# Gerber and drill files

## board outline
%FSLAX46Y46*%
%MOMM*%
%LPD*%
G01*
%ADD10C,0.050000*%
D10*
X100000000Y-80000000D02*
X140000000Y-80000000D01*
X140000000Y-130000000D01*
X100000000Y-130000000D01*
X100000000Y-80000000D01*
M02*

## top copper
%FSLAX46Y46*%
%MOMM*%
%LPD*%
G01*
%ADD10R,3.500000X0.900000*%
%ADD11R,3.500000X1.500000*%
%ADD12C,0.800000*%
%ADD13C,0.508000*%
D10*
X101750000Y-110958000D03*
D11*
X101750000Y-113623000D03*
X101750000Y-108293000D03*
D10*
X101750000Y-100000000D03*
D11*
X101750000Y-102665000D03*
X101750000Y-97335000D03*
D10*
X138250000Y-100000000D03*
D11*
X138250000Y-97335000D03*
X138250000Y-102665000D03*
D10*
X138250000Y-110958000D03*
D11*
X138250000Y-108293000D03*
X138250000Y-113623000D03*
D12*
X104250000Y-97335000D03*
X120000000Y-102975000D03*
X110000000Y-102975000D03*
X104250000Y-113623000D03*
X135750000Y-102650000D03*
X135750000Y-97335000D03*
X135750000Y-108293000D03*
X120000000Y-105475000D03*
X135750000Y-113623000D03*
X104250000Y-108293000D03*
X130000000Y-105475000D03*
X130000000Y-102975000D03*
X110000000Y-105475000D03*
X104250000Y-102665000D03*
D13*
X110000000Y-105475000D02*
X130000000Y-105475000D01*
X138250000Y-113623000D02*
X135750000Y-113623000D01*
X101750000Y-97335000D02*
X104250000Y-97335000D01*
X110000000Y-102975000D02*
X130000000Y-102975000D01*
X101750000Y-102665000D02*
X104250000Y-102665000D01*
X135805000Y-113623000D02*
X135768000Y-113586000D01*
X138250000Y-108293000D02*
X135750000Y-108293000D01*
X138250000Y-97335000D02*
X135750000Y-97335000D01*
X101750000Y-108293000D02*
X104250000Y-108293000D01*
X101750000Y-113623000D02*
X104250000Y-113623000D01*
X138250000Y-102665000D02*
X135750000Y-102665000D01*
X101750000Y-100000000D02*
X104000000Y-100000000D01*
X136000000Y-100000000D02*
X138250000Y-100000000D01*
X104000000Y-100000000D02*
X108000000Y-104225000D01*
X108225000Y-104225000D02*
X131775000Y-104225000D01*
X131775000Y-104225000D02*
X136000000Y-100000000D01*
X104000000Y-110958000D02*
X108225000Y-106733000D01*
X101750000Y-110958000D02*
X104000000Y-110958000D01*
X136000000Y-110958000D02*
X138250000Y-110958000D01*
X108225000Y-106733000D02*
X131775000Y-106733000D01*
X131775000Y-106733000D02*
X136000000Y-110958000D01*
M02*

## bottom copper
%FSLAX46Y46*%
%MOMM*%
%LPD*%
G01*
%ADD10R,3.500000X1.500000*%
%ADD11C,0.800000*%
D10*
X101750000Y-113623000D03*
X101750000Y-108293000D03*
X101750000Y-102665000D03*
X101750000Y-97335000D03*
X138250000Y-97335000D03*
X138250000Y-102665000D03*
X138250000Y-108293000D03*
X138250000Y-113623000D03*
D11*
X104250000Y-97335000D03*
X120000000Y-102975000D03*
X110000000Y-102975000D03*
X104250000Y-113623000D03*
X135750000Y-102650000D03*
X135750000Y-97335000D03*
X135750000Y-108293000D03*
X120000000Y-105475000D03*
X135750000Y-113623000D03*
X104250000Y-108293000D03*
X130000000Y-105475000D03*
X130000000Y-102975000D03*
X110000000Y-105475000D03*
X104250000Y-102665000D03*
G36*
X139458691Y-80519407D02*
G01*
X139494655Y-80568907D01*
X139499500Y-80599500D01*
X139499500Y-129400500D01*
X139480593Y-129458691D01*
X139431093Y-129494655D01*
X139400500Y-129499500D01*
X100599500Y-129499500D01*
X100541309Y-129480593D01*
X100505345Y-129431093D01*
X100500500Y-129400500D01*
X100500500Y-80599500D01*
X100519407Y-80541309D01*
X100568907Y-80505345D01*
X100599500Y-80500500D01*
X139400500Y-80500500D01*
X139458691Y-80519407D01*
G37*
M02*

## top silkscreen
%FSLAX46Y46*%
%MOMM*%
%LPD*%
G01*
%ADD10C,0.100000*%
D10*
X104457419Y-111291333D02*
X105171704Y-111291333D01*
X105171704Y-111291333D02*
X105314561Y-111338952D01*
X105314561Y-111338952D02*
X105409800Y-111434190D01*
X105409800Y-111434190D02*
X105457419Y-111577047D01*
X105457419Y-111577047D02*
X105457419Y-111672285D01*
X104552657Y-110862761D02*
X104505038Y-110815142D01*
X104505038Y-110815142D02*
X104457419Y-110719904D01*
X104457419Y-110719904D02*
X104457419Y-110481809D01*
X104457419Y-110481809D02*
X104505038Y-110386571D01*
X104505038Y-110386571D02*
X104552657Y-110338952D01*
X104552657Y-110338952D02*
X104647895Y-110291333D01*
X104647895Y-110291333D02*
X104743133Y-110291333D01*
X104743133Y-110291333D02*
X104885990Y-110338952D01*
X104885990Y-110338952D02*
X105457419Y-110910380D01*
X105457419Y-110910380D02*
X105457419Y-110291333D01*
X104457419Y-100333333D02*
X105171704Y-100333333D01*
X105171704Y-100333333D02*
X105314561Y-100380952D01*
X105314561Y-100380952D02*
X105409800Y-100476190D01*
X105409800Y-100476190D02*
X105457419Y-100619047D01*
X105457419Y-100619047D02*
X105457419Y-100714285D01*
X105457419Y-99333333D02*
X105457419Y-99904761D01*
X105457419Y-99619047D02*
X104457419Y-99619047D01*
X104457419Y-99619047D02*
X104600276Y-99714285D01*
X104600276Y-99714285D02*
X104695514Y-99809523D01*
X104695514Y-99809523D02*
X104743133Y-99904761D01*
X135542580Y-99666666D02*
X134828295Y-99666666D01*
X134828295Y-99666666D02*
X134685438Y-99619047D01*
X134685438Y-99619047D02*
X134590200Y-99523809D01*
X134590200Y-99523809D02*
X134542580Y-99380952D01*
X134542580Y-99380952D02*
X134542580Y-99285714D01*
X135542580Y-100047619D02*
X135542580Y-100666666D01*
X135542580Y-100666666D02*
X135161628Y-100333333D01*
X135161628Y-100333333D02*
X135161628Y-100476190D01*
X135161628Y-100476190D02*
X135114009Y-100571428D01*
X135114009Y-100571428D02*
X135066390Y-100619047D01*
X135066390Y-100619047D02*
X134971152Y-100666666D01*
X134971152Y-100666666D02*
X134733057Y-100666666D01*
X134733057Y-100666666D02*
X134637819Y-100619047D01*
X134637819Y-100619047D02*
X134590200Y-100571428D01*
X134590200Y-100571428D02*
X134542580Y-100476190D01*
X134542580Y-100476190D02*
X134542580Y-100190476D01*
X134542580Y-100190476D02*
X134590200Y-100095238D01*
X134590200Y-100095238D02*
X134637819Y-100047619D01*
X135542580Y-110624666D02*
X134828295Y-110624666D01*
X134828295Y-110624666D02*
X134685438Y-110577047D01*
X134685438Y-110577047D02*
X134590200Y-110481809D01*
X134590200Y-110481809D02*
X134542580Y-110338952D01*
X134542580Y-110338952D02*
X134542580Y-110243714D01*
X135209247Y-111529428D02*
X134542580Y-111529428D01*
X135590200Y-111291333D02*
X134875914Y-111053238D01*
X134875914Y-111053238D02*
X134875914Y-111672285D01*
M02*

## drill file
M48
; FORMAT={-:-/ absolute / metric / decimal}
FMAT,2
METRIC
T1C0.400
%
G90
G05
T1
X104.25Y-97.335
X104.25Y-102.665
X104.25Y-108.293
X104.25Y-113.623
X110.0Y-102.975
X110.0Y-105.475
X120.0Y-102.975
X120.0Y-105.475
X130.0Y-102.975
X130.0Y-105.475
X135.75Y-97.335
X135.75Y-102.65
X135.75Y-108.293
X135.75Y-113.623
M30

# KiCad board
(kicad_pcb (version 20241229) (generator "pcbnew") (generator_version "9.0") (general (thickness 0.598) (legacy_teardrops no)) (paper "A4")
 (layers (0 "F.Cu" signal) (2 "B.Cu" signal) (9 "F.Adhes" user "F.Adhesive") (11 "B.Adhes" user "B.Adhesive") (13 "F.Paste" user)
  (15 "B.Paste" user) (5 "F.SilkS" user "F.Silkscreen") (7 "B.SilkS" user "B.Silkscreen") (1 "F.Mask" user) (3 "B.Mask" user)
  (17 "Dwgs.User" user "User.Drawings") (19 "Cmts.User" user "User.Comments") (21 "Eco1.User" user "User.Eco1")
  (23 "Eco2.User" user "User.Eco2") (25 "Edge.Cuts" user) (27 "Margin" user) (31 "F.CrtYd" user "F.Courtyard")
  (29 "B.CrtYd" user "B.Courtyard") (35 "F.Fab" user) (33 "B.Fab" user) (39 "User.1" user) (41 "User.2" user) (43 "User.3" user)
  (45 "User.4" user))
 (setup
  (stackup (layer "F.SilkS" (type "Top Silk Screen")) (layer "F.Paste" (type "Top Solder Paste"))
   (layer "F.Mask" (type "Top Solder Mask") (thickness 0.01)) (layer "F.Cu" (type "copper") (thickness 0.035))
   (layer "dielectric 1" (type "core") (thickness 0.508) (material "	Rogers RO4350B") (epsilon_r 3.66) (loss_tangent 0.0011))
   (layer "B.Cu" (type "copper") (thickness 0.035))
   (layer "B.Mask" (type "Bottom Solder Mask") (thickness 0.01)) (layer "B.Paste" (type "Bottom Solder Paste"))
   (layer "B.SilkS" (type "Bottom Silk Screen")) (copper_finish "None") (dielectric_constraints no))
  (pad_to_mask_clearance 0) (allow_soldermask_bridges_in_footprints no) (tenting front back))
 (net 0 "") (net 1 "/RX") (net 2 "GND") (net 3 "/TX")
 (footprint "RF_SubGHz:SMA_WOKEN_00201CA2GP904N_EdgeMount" (layer "F.Cu") (at 100 110.958 90)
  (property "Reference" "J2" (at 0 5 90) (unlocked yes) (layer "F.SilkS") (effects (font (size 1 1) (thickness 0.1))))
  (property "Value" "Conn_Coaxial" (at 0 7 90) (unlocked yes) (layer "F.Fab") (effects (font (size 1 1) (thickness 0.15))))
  (pad "1" smd rect (at 0 1.75 90) (size 0.9 3.5) (layers "F.Cu" "F.Mask") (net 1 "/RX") (thermal_bridge_angle 45))
  (pad "2" smd rect (at -2.665 1.75 90) (size 1.5 3.5) (layers "F.Cu" "F.Mask") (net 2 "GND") (thermal_bridge_angle 45))
  (pad "2" smd rect (at -2.665 1.75 90) (size 1.5 3.5) (layers "B.Cu" "B.Mask") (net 2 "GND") (thermal_bridge_angle 45))
  (pad "2" smd rect (at 2.665 1.75 90) (size 1.5 3.5) (layers "F.Cu" "F.Mask") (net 2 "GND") (thermal_bridge_angle 45))
  (pad "2" smd rect (at 2.665 1.75 90) (size 1.5 3.5) (layers "B.Cu" "B.Mask") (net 2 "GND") (thermal_bridge_angle 45)))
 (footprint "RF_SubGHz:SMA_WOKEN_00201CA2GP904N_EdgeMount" (layer "F.Cu") (at 100 100 90)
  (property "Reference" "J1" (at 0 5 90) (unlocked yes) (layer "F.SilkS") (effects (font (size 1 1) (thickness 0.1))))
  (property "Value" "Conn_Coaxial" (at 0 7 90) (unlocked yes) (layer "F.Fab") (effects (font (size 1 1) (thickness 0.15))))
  (pad "1" smd rect (at 0 1.75 90) (size 0.9 3.5) (layers "F.Cu" "F.Mask") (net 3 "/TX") (thermal_bridge_angle 45))
  (pad "2" smd rect (at -2.665 1.75 90) (size 1.5 3.5) (layers "F.Cu" "F.Mask") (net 2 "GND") (thermal_bridge_angle 45))
  (pad "2" smd rect (at -2.665 1.75 90) (size 1.5 3.5) (layers "B.Cu" "B.Mask") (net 2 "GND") (thermal_bridge_angle 45))
  (pad "2" smd rect (at 2.665 1.75 90) (size 1.5 3.5) (layers "F.Cu" "F.Mask") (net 2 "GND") (thermal_bridge_angle 45))
  (pad "2" smd rect (at 2.665 1.75 90) (size 1.5 3.5) (layers "B.Cu" "B.Mask") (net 2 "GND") (thermal_bridge_angle 45)))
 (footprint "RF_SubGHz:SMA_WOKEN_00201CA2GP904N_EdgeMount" (layer "F.Cu") (at 140 100 -90)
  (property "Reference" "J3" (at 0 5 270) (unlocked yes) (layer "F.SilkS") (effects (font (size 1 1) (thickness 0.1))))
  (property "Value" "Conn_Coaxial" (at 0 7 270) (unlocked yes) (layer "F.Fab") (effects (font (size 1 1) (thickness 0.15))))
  (pad "1" smd rect (at 0 1.75 270) (size 0.9 3.5) (layers "F.Cu" "F.Mask") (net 3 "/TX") (thermal_bridge_angle 45))
  (pad "2" smd rect (at -2.665 1.75 270) (size 1.5 3.5) (layers "F.Cu" "F.Mask") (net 2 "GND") (thermal_bridge_angle 45))
  (pad "2" smd rect (at -2.665 1.75 270) (size 1.5 3.5) (layers "B.Cu" "B.Mask") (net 2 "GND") (thermal_bridge_angle 45))
  (pad "2" smd rect (at 2.665 1.75 270) (size 1.5 3.5) (layers "F.Cu" "F.Mask") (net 2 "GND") (thermal_bridge_angle 45))
  (pad "2" smd rect (at 2.665 1.75 270) (size 1.5 3.5) (layers "B.Cu" "B.Mask") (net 2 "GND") (thermal_bridge_angle 45)))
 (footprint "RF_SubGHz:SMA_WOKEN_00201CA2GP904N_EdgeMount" (layer "F.Cu") (at 140 110.958 -90)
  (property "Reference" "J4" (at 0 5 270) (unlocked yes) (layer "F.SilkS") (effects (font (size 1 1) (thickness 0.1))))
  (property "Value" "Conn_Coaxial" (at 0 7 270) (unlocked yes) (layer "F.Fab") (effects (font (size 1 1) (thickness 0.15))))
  (pad "1" smd rect (at 0 1.75 270) (size 0.9 3.5) (layers "F.Cu" "F.Mask") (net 1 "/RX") (thermal_bridge_angle 45))
  (pad "2" smd rect (at -2.665 1.75 270) (size 1.5 3.5) (layers "F.Cu" "F.Mask") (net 2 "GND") (thermal_bridge_angle 45))
  (pad "2" smd rect (at -2.665 1.75 270) (size 1.5 3.5) (layers "B.Cu" "B.Mask") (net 2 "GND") (thermal_bridge_angle 45))
  (pad "2" smd rect (at 2.665 1.75 270) (size 1.5 3.5) (layers "F.Cu" "F.Mask") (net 2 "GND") (thermal_bridge_angle 45))
  (pad "2" smd rect (at 2.665 1.75 270) (size 1.5 3.5) (layers "B.Cu" "B.Mask") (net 2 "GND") (thermal_bridge_angle 45)))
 (gr_rect (start 100 80) (end 140 130) (stroke (width 0.05) (type solid)) (fill no) (layer "Edge.Cuts"))
 (segment (start 110 105.475) (end 130 105.475) (width 0.508) (layer "F.Cu") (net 2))
 (segment (start 138.25 113.623) (end 135.75 113.623) (width 0.508) (layer "F.Cu") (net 2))
 (segment (start 101.75 97.335) (end 104.25 97.335) (width 0.508) (layer "F.Cu") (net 2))
 (segment (start 110 102.975) (end 130 102.975) (width 0.508) (layer "F.Cu") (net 2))
 (segment (start 101.75 102.665) (end 104.25 102.665) (width 0.508) (layer "F.Cu") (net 2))
 (segment (start 135.805 113.623) (end 135.768 113.586) (width 0.508) (layer "F.Cu") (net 2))
 (segment (start 138.25 108.293) (end 135.75 108.293) (width 0.508) (layer "F.Cu") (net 2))
 (segment (start 138.25 97.335) (end 135.75 97.335) (width 0.508) (layer "F.Cu") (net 2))
 (segment (start 101.75 108.293) (end 104.25 108.293) (width 0.508) (layer "F.Cu") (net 2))
 (segment (start 101.75 113.623) (end 104.25 113.623) (width 0.508) (layer "F.Cu") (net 2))
 (segment (start 138.25 102.665) (end 135.75 102.665) (width 0.508) (layer "F.Cu") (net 2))
 (via (at 104.25 97.335) (size 0.8) (drill 0.4) (layers "F.Cu" "B.Cu") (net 2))
 (via (at 120 102.975) (size 0.8) (drill 0.4) (layers "F.Cu" "B.Cu") (free yes) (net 2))
 (via (at 110 102.975) (size 0.8) (drill 0.4) (layers "F.Cu" "B.Cu") (free yes) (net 2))
 (via (at 104.25 113.623) (size 0.8) (drill 0.4) (layers "F.Cu" "B.Cu") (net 2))
 (via (at 135.75 102.65) (size 0.8) (drill 0.4) (layers "F.Cu" "B.Cu") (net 2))
 (via (at 135.75 97.335) (size 0.8) (drill 0.4) (layers "F.Cu" "B.Cu") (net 2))
 (via (at 135.75 108.293) (size 0.8) (drill 0.4) (layers "F.Cu" "B.Cu") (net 2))
 (via (at 120 105.475) (size 0.8) (drill 0.4) (layers "F.Cu" "B.Cu") (free yes) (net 2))
 (via (at 135.75 113.623) (size 0.8) (drill 0.4) (layers "F.Cu" "B.Cu") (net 2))
 (via (at 104.25 108.293) (size 0.8) (drill 0.4) (layers "F.Cu" "B.Cu") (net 2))
 (via (at 130 105.475) (size 0.8) (drill 0.4) (layers "F.Cu" "B.Cu") (free yes) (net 2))
 (via (at 130 102.975) (size 0.8) (drill 0.4) (layers "F.Cu" "B.Cu") (free yes) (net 2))
 (via (at 110 105.475) (size 0.8) (drill 0.4) (layers "F.Cu" "B.Cu") (free yes) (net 2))
 (via (at 104.25 102.665) (size 0.8) (drill 0.4) (layers "F.Cu" "B.Cu") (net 2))
 (segment (start 101.75 100) (end 104 100) (width 0.508) (layer "F.Cu") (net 3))
 (segment (start 136 100) (end 138.25 100) (width 0.508) (layer "F.Cu") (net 3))
 (segment (start 104 100) (end 108 104.225) (width 0.508) (layer "F.Cu") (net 3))
 (segment (start 108.225 104.225) (end 131.775 104.225) (width 0.508) (layer "F.Cu") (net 3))
 (segment (start 131.775 104.225) (end 136 100) (width 0.508) (layer "F.Cu") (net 3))
 (segment (start 104 110.958) (end 108.225 106.733) (width 0.508) (layer "F.Cu") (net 1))
 (segment (start 101.75 110.958) (end 104 110.958) (width 0.508) (layer "F.Cu") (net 1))
 (segment (start 136 110.958) (end 138.25 110.958) (width 0.508) (layer "F.Cu") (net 1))
 (segment (start 108.225 106.733) (end 131.775 106.733) (width 0.508) (layer "F.Cu") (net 1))
 (segment (start 131.775 106.733) (end 136 110.958) (width 0.508) (layer "F.Cu") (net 1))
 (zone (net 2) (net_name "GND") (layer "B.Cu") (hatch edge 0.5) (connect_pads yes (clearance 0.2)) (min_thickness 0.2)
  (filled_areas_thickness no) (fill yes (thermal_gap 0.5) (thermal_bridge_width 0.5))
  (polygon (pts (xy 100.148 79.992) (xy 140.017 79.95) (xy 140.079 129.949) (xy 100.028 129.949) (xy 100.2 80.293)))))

